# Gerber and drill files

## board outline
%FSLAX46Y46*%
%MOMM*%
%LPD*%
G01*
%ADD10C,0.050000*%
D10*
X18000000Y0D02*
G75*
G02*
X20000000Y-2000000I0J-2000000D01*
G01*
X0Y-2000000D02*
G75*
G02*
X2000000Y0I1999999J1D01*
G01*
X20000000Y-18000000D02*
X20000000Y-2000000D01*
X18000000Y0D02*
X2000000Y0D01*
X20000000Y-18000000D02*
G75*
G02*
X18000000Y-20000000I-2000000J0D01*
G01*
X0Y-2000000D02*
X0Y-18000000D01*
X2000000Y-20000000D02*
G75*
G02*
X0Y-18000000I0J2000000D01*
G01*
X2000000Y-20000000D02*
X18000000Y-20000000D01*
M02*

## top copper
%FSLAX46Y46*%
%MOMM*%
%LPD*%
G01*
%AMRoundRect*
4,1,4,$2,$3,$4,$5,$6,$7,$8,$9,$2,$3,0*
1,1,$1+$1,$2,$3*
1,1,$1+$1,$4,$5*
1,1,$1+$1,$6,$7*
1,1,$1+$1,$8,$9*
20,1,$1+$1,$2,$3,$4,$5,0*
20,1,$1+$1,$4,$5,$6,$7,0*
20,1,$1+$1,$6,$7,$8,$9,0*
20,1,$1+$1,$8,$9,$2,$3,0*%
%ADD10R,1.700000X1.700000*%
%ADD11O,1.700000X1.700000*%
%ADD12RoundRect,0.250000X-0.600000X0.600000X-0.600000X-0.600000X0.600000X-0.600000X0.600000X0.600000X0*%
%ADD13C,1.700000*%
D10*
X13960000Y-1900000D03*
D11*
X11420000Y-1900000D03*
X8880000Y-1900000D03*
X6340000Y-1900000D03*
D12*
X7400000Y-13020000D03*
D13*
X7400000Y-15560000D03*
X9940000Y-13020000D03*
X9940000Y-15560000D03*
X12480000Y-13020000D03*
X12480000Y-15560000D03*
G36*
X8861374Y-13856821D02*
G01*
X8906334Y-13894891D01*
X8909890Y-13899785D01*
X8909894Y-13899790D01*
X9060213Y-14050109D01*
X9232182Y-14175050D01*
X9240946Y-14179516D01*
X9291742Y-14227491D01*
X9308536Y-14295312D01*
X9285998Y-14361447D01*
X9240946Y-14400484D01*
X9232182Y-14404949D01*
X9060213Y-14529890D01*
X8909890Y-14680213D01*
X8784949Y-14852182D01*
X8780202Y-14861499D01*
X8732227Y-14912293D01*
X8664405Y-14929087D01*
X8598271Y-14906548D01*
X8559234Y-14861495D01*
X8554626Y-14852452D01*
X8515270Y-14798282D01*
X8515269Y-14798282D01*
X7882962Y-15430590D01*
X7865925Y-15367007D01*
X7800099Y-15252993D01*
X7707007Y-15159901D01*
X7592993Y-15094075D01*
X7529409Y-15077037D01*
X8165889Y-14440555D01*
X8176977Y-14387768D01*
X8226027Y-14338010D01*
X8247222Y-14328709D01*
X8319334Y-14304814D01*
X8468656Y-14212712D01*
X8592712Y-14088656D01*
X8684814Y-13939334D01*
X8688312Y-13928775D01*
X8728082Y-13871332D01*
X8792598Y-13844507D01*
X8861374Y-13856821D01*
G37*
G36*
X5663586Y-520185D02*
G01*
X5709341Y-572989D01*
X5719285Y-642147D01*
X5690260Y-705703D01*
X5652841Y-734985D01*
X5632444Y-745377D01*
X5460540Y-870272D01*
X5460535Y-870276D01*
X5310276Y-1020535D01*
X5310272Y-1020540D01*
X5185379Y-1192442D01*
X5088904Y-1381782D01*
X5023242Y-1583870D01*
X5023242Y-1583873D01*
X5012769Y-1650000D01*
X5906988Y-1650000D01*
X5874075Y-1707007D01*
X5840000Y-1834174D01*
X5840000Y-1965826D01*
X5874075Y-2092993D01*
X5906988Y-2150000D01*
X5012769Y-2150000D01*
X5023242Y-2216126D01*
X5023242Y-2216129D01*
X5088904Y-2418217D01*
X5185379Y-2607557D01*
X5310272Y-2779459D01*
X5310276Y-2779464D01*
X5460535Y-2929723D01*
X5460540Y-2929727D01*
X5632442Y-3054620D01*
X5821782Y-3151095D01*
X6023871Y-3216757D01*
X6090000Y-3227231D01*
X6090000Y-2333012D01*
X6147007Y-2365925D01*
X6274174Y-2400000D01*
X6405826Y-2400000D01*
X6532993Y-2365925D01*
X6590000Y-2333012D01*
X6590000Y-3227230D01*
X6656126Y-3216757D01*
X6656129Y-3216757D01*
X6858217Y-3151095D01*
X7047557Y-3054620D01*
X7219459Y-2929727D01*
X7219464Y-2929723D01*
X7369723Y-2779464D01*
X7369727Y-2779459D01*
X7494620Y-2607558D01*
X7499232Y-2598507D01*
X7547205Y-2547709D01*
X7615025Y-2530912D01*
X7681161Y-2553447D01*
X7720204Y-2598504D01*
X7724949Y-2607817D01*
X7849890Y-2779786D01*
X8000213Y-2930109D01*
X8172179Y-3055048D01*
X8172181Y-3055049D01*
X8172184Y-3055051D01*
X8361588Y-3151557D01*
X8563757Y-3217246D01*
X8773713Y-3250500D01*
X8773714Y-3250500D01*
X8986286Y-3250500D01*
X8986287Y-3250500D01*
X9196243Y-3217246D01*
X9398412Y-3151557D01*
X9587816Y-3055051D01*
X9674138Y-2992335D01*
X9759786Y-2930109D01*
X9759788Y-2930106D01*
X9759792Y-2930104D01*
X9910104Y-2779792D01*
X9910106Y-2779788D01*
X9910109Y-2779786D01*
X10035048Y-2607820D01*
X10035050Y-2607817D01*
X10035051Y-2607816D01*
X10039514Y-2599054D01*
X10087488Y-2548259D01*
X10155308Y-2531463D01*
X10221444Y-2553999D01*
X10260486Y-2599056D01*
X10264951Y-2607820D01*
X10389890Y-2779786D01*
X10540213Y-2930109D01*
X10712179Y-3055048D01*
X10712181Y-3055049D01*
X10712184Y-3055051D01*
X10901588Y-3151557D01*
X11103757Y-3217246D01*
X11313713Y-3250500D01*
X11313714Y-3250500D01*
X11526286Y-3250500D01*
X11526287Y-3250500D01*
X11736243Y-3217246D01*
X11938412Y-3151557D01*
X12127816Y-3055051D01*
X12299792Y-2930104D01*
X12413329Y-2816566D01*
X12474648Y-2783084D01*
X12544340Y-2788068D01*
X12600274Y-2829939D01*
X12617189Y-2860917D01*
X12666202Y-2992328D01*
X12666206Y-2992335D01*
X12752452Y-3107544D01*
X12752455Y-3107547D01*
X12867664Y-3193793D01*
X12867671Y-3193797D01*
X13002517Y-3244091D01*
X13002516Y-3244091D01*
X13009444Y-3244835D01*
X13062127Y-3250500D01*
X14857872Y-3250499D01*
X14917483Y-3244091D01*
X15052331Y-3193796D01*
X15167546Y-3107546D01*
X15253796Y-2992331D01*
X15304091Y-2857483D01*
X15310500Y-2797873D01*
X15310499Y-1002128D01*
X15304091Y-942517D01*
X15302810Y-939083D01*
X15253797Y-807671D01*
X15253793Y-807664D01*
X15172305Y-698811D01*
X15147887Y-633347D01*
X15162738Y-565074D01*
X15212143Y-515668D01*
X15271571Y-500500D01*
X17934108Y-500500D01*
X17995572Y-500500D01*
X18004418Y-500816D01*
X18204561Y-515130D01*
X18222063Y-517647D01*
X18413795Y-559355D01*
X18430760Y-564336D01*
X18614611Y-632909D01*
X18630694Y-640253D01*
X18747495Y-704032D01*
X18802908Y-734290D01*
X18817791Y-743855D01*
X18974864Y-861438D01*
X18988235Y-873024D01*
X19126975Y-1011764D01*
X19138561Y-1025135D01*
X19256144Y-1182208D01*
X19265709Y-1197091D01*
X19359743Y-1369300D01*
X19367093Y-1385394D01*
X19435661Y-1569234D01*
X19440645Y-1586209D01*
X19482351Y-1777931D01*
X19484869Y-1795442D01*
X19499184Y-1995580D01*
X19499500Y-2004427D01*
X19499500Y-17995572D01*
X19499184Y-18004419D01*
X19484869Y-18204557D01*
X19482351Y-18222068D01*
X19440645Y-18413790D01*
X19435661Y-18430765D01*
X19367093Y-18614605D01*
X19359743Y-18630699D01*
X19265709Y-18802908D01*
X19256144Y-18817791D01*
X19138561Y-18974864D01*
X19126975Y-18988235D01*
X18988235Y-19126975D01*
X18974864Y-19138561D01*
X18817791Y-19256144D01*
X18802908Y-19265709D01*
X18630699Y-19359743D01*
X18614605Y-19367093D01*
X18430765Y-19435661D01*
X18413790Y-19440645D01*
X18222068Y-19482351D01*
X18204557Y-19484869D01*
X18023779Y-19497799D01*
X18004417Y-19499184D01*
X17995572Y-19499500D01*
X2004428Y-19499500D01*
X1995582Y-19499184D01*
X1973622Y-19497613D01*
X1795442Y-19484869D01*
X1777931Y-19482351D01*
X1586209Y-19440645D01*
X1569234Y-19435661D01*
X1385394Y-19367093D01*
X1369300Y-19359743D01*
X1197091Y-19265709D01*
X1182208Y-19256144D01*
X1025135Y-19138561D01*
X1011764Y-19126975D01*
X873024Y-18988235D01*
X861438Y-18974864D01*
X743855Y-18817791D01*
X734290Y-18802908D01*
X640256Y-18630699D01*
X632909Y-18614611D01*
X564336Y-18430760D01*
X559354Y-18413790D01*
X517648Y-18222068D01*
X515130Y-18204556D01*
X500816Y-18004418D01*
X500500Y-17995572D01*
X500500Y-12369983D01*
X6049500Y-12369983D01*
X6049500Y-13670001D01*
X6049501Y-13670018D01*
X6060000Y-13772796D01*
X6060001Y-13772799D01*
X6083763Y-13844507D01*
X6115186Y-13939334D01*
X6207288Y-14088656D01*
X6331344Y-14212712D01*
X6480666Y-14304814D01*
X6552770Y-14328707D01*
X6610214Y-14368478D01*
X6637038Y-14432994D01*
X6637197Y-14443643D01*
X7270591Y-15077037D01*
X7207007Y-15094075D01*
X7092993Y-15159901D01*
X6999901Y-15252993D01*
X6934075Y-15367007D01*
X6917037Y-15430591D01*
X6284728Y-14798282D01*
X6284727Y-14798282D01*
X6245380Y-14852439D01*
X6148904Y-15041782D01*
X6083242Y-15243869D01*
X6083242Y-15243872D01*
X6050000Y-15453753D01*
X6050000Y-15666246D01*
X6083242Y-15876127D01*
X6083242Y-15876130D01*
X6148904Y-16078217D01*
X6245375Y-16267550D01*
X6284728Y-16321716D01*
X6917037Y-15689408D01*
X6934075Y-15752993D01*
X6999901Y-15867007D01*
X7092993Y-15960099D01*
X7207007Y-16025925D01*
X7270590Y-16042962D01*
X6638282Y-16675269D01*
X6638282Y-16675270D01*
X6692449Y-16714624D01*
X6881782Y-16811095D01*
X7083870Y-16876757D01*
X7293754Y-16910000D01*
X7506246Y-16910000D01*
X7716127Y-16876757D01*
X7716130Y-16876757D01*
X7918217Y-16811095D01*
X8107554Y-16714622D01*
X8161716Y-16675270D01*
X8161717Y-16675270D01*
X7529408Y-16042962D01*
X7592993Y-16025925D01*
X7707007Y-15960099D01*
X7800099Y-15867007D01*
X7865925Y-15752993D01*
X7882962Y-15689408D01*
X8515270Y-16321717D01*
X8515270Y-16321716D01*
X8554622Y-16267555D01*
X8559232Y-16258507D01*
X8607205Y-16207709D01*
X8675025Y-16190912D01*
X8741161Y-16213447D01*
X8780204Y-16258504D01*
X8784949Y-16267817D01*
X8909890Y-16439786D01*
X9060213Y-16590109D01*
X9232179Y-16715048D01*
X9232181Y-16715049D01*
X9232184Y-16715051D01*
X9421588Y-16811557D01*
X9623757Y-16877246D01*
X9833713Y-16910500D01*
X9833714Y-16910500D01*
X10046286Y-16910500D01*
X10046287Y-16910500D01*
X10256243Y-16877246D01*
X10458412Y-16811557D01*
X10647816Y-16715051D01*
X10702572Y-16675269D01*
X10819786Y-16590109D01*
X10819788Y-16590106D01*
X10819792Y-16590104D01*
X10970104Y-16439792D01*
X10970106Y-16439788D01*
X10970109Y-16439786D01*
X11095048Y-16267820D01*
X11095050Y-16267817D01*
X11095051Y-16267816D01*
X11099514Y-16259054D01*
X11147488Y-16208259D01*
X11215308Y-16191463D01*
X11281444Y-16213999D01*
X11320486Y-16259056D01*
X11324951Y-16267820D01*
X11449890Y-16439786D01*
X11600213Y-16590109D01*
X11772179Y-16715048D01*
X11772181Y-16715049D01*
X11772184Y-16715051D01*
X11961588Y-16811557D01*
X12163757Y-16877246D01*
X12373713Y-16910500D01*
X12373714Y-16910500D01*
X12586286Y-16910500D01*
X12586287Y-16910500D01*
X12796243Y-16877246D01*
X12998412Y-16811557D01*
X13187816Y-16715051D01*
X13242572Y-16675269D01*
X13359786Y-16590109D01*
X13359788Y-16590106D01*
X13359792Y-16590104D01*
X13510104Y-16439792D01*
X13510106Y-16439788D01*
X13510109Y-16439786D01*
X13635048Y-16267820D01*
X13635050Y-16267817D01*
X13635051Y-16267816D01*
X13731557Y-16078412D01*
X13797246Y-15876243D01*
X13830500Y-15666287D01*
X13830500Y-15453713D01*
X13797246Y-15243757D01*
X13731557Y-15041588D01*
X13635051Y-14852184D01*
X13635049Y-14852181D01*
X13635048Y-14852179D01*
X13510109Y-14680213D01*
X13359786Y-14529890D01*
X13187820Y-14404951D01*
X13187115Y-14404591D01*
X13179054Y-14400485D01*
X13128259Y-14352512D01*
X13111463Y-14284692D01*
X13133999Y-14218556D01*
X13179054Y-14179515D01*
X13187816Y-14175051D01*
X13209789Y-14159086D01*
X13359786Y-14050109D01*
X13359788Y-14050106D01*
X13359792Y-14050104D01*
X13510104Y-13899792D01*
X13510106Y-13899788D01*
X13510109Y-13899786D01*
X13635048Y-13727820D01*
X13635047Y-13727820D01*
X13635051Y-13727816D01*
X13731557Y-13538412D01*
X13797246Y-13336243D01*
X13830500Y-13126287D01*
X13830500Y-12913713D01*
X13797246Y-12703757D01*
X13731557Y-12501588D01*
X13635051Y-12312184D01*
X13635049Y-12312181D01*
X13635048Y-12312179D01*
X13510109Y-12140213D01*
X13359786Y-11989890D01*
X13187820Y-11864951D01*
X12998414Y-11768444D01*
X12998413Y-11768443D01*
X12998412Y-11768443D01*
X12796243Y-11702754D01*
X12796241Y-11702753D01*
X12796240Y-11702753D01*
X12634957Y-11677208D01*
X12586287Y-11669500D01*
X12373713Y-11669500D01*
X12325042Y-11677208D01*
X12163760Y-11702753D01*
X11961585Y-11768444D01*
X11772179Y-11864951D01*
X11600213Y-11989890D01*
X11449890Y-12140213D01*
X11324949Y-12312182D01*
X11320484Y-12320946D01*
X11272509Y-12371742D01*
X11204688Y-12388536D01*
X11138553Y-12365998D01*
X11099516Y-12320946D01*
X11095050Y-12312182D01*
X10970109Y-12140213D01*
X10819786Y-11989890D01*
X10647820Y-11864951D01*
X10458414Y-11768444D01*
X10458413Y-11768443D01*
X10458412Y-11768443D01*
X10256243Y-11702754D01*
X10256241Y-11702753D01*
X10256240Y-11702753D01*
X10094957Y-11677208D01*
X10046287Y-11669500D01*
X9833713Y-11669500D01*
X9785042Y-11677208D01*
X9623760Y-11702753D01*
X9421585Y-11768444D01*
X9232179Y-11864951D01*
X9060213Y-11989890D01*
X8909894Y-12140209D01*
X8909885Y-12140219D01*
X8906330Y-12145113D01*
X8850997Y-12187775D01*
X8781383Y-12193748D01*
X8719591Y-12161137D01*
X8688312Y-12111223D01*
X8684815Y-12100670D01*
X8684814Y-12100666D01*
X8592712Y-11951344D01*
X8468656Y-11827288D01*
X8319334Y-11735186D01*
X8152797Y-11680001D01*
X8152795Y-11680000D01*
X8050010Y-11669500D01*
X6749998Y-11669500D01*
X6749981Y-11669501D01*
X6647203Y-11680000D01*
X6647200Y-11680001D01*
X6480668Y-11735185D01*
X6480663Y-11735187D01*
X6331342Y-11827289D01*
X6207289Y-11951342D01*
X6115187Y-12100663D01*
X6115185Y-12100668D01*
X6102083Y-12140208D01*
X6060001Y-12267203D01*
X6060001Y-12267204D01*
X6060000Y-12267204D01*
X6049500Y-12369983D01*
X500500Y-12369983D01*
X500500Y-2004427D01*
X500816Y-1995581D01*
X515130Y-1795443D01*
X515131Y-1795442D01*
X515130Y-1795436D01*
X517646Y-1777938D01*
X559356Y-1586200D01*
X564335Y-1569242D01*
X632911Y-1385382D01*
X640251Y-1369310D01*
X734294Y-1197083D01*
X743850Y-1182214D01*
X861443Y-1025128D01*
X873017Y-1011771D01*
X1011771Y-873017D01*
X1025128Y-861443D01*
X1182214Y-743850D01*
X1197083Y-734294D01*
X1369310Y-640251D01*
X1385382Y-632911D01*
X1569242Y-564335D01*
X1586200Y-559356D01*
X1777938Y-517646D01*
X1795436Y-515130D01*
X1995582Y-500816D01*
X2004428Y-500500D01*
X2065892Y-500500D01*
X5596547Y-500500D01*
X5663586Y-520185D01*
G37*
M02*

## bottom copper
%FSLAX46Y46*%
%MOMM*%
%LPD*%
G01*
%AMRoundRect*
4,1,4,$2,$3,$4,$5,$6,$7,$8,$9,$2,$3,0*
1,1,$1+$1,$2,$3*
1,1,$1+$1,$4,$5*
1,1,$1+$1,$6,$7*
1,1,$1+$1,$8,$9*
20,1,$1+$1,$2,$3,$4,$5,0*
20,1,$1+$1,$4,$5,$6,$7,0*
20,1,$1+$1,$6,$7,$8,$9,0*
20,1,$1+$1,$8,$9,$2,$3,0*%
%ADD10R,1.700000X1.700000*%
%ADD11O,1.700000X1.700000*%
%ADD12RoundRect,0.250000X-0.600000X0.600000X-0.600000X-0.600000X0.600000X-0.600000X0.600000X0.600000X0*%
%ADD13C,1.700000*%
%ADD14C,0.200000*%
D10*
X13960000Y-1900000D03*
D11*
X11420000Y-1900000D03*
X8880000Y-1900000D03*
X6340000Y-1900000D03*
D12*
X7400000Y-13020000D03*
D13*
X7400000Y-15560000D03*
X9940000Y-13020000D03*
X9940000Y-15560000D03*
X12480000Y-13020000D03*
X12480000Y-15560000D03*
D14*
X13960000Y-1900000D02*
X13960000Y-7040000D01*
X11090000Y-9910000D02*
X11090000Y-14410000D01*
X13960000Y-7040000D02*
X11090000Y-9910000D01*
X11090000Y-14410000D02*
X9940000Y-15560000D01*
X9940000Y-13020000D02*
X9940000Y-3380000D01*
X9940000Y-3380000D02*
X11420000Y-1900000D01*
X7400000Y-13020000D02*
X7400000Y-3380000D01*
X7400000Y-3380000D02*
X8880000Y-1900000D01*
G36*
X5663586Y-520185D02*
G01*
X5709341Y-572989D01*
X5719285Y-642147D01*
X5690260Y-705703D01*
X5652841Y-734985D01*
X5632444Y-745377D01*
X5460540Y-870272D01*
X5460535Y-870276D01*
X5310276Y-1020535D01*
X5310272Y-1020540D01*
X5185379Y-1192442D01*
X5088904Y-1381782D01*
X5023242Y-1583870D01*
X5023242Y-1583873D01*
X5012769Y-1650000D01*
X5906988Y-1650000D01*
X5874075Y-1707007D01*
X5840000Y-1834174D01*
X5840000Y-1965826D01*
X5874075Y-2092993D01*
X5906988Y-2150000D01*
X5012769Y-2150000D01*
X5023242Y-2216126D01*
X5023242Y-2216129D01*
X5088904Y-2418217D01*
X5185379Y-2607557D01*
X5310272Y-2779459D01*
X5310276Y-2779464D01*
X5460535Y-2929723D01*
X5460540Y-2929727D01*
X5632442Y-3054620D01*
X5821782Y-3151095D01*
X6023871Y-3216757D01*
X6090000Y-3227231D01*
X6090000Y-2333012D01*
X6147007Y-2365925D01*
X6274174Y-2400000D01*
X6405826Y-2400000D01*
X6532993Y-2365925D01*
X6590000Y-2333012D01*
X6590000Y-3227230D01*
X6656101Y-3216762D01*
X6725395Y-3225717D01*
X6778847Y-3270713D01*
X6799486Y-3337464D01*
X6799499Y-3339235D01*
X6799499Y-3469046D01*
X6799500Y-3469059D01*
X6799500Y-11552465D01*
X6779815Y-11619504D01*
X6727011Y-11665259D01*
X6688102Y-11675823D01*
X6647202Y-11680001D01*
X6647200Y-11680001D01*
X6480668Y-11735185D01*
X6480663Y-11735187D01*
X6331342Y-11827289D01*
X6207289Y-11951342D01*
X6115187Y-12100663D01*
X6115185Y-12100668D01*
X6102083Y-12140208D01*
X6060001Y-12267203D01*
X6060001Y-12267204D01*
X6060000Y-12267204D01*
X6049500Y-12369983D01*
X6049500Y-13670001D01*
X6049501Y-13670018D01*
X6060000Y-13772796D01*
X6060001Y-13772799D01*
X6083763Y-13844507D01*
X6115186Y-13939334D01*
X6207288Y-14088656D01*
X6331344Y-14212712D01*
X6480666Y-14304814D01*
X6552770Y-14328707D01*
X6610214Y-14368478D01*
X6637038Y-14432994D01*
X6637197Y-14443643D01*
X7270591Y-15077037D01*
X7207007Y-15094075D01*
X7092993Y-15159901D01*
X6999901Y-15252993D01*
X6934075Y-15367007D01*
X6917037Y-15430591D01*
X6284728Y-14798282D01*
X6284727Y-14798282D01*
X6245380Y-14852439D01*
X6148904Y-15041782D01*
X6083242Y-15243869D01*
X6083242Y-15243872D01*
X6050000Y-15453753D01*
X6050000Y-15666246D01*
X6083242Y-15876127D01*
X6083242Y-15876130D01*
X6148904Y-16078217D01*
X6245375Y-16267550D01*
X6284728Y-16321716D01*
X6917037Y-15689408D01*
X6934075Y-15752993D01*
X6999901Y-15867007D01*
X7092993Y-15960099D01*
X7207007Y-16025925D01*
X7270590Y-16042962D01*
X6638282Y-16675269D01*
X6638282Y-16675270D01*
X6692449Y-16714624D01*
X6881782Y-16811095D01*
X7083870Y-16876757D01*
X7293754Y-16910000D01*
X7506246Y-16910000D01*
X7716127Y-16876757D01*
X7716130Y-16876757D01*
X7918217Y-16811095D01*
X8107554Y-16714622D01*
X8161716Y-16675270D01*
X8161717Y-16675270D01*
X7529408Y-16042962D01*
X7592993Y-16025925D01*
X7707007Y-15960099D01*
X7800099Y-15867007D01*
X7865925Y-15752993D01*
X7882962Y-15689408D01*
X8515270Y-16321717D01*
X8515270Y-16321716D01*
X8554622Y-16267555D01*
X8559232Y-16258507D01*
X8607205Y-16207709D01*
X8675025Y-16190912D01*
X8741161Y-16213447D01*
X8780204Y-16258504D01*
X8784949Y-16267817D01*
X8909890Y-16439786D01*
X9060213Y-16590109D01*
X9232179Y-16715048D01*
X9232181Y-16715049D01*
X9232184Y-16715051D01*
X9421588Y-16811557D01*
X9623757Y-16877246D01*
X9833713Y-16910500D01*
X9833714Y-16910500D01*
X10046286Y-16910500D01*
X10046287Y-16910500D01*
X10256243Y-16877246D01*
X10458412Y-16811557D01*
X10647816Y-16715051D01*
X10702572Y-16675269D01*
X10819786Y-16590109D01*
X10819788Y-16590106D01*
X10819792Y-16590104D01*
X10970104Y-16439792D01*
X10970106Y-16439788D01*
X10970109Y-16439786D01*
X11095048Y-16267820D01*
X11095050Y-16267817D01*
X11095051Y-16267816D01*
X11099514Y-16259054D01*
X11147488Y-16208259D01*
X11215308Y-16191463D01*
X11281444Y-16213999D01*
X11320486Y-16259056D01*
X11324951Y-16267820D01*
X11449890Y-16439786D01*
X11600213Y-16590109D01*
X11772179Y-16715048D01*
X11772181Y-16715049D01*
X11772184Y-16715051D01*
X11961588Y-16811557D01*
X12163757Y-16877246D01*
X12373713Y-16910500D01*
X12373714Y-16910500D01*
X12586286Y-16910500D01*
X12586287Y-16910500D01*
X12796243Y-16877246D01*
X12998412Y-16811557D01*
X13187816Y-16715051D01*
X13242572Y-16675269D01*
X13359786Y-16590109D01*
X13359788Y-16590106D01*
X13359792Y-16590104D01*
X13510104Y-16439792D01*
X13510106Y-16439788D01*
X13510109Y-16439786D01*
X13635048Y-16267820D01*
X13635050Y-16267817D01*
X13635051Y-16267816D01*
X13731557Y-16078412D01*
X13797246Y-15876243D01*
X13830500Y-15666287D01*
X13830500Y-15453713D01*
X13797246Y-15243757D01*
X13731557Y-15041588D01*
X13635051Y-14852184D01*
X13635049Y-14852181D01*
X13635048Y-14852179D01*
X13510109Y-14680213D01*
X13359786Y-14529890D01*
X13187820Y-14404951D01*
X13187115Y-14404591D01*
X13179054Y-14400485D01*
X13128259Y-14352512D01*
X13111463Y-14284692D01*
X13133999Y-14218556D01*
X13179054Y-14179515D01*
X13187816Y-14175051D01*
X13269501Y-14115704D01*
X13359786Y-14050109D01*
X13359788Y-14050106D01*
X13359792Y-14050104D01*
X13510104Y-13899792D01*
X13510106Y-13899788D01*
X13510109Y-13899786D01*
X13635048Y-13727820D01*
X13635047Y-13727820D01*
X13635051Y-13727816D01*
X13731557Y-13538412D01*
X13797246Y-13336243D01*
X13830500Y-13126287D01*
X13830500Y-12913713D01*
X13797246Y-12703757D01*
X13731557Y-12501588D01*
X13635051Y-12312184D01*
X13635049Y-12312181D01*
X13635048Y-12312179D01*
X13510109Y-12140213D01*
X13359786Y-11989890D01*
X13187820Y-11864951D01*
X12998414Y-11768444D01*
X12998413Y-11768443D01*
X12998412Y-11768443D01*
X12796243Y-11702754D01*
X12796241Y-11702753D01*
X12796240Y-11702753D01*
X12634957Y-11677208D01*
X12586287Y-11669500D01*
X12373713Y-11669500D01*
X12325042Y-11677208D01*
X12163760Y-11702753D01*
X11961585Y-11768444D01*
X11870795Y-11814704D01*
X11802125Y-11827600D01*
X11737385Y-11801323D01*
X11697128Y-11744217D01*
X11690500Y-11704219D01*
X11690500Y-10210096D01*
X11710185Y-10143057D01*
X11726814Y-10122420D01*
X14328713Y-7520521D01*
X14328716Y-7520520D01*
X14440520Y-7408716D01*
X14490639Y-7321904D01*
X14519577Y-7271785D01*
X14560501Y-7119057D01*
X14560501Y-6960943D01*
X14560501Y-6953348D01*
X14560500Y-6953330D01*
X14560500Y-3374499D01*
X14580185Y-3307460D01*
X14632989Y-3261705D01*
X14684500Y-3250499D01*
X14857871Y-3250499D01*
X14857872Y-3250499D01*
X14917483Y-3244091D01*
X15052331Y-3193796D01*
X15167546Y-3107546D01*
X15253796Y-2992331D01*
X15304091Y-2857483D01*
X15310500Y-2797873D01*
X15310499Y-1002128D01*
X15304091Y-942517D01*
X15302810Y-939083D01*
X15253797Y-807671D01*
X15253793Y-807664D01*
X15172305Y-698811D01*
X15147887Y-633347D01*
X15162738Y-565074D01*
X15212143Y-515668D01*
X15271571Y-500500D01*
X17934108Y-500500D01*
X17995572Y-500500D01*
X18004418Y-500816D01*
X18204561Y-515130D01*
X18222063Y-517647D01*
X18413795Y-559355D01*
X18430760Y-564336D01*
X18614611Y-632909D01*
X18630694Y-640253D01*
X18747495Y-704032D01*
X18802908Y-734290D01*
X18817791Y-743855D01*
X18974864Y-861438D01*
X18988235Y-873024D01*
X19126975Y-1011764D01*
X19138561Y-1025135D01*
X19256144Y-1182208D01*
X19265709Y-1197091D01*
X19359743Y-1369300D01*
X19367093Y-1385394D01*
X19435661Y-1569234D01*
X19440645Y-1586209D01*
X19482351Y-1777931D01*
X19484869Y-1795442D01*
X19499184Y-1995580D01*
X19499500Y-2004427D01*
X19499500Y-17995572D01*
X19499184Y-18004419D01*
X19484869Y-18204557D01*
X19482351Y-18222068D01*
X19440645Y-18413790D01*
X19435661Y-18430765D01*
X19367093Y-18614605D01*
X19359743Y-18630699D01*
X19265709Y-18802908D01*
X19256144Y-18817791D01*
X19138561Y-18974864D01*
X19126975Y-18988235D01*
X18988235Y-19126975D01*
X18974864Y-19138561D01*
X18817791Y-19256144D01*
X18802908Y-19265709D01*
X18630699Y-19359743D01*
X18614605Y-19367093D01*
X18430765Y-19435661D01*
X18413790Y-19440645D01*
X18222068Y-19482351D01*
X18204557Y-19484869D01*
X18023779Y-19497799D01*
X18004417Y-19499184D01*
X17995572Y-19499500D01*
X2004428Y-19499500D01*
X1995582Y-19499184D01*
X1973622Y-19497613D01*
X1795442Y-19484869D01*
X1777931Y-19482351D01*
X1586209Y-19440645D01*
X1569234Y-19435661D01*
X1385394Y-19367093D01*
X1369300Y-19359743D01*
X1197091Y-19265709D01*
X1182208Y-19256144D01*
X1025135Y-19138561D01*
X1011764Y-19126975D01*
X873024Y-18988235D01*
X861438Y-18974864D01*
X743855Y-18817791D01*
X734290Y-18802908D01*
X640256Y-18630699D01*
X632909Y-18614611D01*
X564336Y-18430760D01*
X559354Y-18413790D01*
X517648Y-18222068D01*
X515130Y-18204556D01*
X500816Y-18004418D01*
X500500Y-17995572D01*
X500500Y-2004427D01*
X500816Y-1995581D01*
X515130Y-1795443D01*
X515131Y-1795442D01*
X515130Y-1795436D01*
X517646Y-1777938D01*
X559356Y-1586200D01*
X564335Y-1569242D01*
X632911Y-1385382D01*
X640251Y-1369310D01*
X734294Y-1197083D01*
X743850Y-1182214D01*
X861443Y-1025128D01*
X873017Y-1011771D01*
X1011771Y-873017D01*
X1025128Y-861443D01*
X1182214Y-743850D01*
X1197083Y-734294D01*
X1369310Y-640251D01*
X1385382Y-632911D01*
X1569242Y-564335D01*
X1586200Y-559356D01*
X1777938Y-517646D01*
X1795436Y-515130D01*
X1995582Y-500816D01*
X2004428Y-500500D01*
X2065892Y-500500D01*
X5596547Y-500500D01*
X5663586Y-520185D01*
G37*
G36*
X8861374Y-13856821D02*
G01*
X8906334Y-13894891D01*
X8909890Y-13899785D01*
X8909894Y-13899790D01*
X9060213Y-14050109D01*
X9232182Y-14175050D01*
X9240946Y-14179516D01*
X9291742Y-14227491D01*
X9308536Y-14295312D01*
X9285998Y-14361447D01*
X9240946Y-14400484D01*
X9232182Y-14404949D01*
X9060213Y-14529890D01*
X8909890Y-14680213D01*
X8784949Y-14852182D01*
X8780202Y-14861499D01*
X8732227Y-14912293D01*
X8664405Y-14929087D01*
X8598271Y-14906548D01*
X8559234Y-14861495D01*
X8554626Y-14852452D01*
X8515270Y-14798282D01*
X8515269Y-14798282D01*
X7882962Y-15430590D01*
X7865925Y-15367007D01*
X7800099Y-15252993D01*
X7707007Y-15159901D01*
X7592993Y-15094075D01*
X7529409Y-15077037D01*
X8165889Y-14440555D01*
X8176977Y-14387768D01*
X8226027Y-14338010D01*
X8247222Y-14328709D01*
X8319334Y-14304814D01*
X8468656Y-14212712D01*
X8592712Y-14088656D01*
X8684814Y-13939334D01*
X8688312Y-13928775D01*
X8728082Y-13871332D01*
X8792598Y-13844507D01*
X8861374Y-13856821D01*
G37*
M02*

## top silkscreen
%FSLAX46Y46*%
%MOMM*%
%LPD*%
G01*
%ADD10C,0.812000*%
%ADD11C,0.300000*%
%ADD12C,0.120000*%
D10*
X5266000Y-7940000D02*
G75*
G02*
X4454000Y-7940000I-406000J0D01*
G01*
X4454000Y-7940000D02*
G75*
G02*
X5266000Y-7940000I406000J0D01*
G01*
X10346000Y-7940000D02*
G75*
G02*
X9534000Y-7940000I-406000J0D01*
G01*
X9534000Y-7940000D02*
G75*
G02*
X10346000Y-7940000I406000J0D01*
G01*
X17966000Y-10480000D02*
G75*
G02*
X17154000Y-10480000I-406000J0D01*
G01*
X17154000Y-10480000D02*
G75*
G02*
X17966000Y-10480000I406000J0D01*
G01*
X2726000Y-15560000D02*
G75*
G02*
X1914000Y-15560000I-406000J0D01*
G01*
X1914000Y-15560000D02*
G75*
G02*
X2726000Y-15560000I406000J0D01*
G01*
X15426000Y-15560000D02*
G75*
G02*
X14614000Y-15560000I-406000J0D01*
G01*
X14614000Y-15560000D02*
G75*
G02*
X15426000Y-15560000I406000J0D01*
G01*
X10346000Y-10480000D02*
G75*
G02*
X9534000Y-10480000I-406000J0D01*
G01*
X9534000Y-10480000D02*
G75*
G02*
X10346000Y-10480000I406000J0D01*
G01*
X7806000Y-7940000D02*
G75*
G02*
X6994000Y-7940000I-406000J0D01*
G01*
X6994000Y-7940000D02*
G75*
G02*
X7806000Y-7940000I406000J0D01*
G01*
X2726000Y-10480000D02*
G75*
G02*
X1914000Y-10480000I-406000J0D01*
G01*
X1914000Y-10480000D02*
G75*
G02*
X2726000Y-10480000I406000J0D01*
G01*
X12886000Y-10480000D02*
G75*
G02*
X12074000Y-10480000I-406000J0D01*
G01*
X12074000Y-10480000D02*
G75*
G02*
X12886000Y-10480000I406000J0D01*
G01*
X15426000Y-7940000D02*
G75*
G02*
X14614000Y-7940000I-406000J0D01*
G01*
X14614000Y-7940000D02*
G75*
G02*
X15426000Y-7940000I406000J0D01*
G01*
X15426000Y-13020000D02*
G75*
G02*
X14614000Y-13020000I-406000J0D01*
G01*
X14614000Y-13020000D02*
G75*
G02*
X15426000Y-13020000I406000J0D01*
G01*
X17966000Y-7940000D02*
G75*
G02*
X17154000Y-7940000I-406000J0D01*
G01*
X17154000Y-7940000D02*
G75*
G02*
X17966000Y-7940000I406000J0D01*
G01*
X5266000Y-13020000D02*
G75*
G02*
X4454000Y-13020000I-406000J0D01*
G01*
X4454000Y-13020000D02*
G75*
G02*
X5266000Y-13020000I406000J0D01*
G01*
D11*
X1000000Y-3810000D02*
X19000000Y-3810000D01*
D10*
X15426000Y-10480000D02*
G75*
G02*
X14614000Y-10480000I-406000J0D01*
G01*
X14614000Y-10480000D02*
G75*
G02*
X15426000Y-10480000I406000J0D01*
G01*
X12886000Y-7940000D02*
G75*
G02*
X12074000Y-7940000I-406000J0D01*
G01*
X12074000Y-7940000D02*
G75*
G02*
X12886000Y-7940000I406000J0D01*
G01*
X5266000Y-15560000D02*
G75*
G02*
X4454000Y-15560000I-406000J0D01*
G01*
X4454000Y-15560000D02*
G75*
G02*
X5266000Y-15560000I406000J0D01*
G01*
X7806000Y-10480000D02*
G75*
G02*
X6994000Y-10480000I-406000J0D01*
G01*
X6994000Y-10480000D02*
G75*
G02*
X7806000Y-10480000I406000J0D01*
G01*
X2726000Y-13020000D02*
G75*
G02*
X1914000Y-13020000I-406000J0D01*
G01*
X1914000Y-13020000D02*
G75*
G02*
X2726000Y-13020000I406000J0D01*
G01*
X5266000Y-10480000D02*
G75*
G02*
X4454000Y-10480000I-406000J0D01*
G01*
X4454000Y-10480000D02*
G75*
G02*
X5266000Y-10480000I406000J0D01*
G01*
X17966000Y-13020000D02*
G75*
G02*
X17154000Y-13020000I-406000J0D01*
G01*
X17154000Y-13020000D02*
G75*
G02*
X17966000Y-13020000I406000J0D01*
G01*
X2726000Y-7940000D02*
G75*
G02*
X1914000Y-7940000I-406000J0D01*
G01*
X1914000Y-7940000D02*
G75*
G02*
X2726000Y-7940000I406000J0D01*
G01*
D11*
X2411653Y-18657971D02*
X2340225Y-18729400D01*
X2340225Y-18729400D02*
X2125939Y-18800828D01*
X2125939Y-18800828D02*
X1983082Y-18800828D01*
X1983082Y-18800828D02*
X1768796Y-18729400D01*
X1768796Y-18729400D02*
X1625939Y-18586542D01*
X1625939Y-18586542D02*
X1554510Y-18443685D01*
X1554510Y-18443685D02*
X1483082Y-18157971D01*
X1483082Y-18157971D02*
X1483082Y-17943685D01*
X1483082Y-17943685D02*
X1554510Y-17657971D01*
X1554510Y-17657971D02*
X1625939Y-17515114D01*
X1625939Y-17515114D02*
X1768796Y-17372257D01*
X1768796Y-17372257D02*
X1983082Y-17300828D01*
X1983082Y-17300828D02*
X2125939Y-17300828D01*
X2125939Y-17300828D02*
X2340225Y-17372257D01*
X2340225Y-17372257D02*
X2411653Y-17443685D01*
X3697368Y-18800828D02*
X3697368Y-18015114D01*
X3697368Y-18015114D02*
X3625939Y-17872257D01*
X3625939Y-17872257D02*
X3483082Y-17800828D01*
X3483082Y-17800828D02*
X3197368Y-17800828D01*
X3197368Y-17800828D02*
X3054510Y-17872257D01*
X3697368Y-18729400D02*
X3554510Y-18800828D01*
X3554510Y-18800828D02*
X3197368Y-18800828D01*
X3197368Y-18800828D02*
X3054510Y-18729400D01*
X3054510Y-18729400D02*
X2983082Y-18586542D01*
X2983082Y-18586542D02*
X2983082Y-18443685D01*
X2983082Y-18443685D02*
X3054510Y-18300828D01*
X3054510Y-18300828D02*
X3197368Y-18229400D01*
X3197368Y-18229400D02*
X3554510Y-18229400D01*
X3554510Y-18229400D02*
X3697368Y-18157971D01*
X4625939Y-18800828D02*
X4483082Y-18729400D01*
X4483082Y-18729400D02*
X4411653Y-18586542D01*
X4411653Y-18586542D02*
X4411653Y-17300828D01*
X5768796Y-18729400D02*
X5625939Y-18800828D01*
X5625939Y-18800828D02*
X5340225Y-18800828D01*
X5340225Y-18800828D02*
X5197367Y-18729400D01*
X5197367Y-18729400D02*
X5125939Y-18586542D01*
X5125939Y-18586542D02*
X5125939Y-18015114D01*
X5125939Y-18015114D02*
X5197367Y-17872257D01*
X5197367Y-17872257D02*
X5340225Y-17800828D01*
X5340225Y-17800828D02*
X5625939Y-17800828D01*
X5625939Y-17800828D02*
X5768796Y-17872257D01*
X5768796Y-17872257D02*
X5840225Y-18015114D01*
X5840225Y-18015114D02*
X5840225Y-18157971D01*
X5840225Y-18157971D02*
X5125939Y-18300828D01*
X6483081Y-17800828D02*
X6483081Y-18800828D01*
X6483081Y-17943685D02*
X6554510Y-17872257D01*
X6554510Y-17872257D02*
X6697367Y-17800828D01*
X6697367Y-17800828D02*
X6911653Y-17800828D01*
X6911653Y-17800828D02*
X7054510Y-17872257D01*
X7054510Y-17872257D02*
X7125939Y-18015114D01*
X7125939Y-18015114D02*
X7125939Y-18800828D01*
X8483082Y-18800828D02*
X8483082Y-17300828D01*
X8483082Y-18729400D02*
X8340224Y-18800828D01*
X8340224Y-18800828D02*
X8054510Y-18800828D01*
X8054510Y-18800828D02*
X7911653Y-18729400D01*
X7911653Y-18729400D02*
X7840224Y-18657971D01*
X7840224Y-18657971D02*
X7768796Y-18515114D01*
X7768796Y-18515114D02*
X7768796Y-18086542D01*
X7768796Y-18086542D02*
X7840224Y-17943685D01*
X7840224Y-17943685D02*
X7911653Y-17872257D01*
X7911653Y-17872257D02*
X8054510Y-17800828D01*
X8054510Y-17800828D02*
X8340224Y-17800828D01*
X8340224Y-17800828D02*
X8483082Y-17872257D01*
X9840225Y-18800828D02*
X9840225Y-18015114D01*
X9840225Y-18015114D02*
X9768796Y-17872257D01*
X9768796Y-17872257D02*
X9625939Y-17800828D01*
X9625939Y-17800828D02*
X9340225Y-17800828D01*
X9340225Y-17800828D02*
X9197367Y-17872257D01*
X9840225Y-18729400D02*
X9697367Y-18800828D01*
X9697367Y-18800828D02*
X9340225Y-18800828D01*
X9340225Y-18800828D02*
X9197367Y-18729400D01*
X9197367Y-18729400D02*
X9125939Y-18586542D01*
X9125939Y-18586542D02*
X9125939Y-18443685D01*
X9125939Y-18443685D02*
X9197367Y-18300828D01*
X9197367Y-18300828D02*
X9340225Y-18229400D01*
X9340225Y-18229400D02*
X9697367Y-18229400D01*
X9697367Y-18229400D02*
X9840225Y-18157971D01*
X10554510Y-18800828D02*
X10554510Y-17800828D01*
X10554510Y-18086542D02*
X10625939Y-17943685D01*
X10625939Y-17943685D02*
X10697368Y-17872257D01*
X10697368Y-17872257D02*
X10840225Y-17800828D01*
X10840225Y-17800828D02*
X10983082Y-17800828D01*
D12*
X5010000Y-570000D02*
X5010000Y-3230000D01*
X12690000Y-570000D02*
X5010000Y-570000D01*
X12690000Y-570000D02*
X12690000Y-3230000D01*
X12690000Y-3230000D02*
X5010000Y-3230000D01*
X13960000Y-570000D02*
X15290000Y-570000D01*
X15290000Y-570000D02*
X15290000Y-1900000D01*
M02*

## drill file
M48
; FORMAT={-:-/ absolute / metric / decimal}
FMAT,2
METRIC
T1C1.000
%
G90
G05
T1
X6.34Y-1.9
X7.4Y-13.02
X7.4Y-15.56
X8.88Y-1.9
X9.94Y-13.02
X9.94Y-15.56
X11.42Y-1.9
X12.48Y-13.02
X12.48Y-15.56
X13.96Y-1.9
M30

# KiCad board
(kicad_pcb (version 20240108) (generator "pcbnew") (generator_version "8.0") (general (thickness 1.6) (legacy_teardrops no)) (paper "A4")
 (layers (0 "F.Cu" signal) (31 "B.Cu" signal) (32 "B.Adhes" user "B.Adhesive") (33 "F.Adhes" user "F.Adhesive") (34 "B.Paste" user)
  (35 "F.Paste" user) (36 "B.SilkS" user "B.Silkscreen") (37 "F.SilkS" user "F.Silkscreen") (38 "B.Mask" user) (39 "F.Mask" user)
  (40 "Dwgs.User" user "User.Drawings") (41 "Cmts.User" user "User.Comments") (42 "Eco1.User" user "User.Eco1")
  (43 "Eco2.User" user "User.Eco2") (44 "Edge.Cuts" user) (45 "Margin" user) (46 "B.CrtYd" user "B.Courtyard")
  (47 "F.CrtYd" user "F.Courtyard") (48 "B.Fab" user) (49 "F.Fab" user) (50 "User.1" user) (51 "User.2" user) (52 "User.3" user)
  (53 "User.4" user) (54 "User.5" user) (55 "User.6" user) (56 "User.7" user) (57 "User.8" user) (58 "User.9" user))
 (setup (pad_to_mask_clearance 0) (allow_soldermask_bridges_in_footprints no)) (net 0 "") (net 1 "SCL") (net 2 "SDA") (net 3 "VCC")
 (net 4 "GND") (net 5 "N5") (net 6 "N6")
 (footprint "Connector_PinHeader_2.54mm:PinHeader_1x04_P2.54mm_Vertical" (layer "F.Cu") (at 13.96 1.9 -90)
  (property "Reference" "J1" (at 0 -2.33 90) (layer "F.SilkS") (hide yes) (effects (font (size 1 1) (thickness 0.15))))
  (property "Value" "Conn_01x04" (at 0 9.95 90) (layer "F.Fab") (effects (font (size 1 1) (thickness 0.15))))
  (fp_line (start -1.33 8.95) (end 1.33 8.95) (stroke (width 0.12) (type solid)) (layer "F.SilkS"))
  (fp_line (start -1.33 1.27) (end -1.33 8.95) (stroke (width 0.12) (type solid)) (layer "F.SilkS"))
  (fp_line (start -1.33 1.27) (end 1.33 1.27) (stroke (width 0.12) (type solid)) (layer "F.SilkS"))
  (fp_line (start 1.33 1.27) (end 1.33 8.95) (stroke (width 0.12) (type solid)) (layer "F.SilkS"))
  (fp_line (start -1.33 0) (end -1.33 -1.33) (stroke (width 0.12) (type solid)) (layer "F.SilkS"))
  (fp_line (start -1.33 -1.33) (end 0 -1.33) (stroke (width 0.12) (type solid)) (layer "F.SilkS"))
  (pad "1" thru_hole rect (at 0 0 270) (size 1.7 1.7) (drill 1) (layers "*.Cu" "*.Mask") (remove_unused_layers no) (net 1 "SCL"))
  (pad "2" thru_hole oval (at 0 2.54 270) (size 1.7 1.7) (drill 1) (layers "*.Cu" "*.Mask") (remove_unused_layers no) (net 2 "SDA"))
  (pad "3" thru_hole oval (at 0 5.08 270) (size 1.7 1.7) (drill 1) (layers "*.Cu" "*.Mask") (remove_unused_layers no) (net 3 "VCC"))
  (pad "4" thru_hole oval (at 0 7.62 270) (size 1.7 1.7) (drill 1) (layers "*.Cu" "*.Mask") (remove_unused_layers no) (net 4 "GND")))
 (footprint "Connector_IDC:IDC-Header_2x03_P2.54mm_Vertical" (layer "B.Cu") (at 7.4 13.02 -90)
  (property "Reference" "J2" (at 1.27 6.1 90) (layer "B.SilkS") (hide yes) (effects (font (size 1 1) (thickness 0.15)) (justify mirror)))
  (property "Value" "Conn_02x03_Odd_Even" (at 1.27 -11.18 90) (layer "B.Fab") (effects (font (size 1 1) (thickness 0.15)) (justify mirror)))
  (pad "1" thru_hole roundrect (at 0 0 270) (size 1.7 1.7) (drill 1) (layers "*.Cu" "*.Mask") (remove_unused_layers no)
   (roundrect_rratio 0.147059) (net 3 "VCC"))
  (pad "2" thru_hole circle (at 2.54 0 270) (size 1.7 1.7) (drill 1) (layers "*.Cu" "*.Mask") (remove_unused_layers no) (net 4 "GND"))
  (pad "3" thru_hole circle (at 0 -2.54 270) (size 1.7 1.7) (drill 1) (layers "*.Cu" "*.Mask") (remove_unused_layers no) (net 2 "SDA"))
  (pad "4" thru_hole circle (at 2.54 -2.54 270) (size 1.7 1.7) (drill 1) (layers "*.Cu" "*.Mask") (remove_unused_layers no) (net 1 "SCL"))
  (pad "5" thru_hole circle (at 0 -5.08 270) (size 1.7 1.7) (drill 1) (layers "*.Cu" "*.Mask") (remove_unused_layers no) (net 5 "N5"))
  (pad "6" thru_hole circle (at 2.54 -5.08 270) (size 1.7 1.7) (drill 1) (layers "*.Cu" "*.Mask") (remove_unused_layers no) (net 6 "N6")))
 (gr_circle (center 4.86 7.94) (end 5.622 7.94) (stroke (width 0.1) (type solid)) (fill solid) (layer "F.SilkS"))
 (gr_circle (center 9.94 7.94) (end 10.702 7.94) (stroke (width 0.1) (type solid)) (fill solid) (layer "F.SilkS"))
 (gr_circle (center 17.56 10.48) (end 18.322 10.48) (stroke (width 0.1) (type solid)) (fill solid) (layer "F.SilkS"))
 (gr_circle (center 2.32 15.56) (end 3.082 15.56) (stroke (width 0.1) (type solid)) (fill solid) (layer "F.SilkS"))
 (gr_circle (center 15.02 15.56) (end 15.782 15.56) (stroke (width 0.1) (type solid)) (fill solid) (layer "F.SilkS"))
 (gr_circle (center 9.94 10.48) (end 10.702 10.48) (stroke (width 0.1) (type solid)) (fill solid) (layer "F.SilkS"))
 (gr_circle (center 7.4 7.94) (end 8.162 7.94) (stroke (width 0.1) (type solid)) (fill solid) (layer "F.SilkS"))
 (gr_circle (center 2.32 10.48) (end 3.082 10.48) (stroke (width 0.1) (type solid)) (fill solid) (layer "F.SilkS"))
 (gr_circle (center 12.48 10.48) (end 13.242 10.48) (stroke (width 0.1) (type solid)) (fill solid) (layer "F.SilkS"))
 (gr_circle (center 15.02 7.94) (end 15.782 7.94) (stroke (width 0.1) (type solid)) (fill solid) (layer "F.SilkS"))
 (gr_circle (center 15.02 13.02) (end 15.782 13.02) (stroke (width 0.1) (type solid)) (fill solid) (layer "F.SilkS"))
 (gr_circle (center 17.56 7.94) (end 18.322 7.94) (stroke (width 0.1) (type solid)) (fill solid) (layer "F.SilkS"))
 (gr_circle (center 4.86 13.02) (end 5.622 13.02) (stroke (width 0.1) (type solid)) (fill solid) (layer "F.SilkS"))
 (gr_line (start 1 3.81) (end 19 3.81) (stroke (width 0.3) (type default)) (layer "F.SilkS"))
 (gr_circle (center 15.02 10.48) (end 15.782 10.48) (stroke (width 0.1) (type solid)) (fill solid) (layer "F.SilkS"))
 (gr_circle (center 12.48 7.94) (end 13.242 7.94) (stroke (width 0.1) (type solid)) (fill solid) (layer "F.SilkS"))
 (gr_circle (center 4.86 15.56) (end 5.622 15.56) (stroke (width 0.1) (type solid)) (fill solid) (layer "F.SilkS"))
 (gr_circle (center 7.4 10.48) (end 8.162 10.48) (stroke (width 0.1) (type solid)) (fill solid) (layer "F.SilkS"))
 (gr_circle (center 2.32 13.02) (end 3.082 13.02) (stroke (width 0.1) (type solid)) (fill solid) (layer "F.SilkS"))
 (gr_circle (center 4.86 10.48) (end 5.622 10.48) (stroke (width 0.1) (type solid)) (fill solid) (layer "F.SilkS"))
 (gr_circle (center 17.56 13.02) (end 18.322 13.02) (stroke (width 0.1) (type solid)) (fill solid) (layer "F.SilkS"))
 (gr_circle (center 2.32 7.94) (end 3.082 7.94) (stroke (width 0.1) (type solid)) (fill solid) (layer "F.SilkS"))
 (gr_arc (start 18 0) (mid 19.414214 0.585786) (end 20 2) (stroke (width 0.05) (type default)) (layer "Edge.Cuts"))
 (gr_arc (start 0 2) (mid 0.585786 0.585786) (end 2 0) (stroke (width 0.05) (type default)) (layer "Edge.Cuts"))
 (gr_line (start 20 18) (end 20 2) (stroke (width 0.05) (type default)) (layer "Edge.Cuts"))
 (gr_line (start 18 0) (end 2 0) (stroke (width 0.05) (type default)) (layer "Edge.Cuts"))
 (gr_arc (start 20 18) (mid 19.414214 19.414214) (end 18 20) (stroke (width 0.05) (type default)) (layer "Edge.Cuts"))
 (gr_line (start 0 2) (end 0 18) (stroke (width 0.05) (type default)) (layer "Edge.Cuts"))
 (gr_arc (start 2 20) (mid 0.585786 19.414214) (end 0 18) (stroke (width 0.05) (type default)) (layer "Edge.Cuts"))
 (gr_line (start 2 20) (end 18 20) (stroke (width 0.05) (type default)) (layer "Edge.Cuts"))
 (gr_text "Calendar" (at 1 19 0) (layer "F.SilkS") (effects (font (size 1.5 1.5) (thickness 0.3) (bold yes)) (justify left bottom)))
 (segment (start 13.96 1.9) (end 13.96 7.04) (width 0.2) (layer "B.Cu") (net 1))
 (segment (start 11.09 9.91) (end 11.09 14.41) (width 0.2) (layer "B.Cu") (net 1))
 (segment (start 13.96 7.04) (end 11.09 9.91) (width 0.2) (layer "B.Cu") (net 1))
 (segment (start 11.09 14.41) (end 9.94 15.56) (width 0.2) (layer "B.Cu") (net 1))
 (segment (start 9.94 13.02) (end 9.94 3.38) (width 0.2) (layer "B.Cu") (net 2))
 (segment (start 9.94 3.38) (end 11.42 1.9) (width 0.2) (layer "B.Cu") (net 2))
 (segment (start 7.4 13.02) (end 7.4 3.38) (width 0.2) (layer "B.Cu") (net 3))
 (segment (start 7.4 3.38) (end 8.88 1.9) (width 0.2) (layer "B.Cu") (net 3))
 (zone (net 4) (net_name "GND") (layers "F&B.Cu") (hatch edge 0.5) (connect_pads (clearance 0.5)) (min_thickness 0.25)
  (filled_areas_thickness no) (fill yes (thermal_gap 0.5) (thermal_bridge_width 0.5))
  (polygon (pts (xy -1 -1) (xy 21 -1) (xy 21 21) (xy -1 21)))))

